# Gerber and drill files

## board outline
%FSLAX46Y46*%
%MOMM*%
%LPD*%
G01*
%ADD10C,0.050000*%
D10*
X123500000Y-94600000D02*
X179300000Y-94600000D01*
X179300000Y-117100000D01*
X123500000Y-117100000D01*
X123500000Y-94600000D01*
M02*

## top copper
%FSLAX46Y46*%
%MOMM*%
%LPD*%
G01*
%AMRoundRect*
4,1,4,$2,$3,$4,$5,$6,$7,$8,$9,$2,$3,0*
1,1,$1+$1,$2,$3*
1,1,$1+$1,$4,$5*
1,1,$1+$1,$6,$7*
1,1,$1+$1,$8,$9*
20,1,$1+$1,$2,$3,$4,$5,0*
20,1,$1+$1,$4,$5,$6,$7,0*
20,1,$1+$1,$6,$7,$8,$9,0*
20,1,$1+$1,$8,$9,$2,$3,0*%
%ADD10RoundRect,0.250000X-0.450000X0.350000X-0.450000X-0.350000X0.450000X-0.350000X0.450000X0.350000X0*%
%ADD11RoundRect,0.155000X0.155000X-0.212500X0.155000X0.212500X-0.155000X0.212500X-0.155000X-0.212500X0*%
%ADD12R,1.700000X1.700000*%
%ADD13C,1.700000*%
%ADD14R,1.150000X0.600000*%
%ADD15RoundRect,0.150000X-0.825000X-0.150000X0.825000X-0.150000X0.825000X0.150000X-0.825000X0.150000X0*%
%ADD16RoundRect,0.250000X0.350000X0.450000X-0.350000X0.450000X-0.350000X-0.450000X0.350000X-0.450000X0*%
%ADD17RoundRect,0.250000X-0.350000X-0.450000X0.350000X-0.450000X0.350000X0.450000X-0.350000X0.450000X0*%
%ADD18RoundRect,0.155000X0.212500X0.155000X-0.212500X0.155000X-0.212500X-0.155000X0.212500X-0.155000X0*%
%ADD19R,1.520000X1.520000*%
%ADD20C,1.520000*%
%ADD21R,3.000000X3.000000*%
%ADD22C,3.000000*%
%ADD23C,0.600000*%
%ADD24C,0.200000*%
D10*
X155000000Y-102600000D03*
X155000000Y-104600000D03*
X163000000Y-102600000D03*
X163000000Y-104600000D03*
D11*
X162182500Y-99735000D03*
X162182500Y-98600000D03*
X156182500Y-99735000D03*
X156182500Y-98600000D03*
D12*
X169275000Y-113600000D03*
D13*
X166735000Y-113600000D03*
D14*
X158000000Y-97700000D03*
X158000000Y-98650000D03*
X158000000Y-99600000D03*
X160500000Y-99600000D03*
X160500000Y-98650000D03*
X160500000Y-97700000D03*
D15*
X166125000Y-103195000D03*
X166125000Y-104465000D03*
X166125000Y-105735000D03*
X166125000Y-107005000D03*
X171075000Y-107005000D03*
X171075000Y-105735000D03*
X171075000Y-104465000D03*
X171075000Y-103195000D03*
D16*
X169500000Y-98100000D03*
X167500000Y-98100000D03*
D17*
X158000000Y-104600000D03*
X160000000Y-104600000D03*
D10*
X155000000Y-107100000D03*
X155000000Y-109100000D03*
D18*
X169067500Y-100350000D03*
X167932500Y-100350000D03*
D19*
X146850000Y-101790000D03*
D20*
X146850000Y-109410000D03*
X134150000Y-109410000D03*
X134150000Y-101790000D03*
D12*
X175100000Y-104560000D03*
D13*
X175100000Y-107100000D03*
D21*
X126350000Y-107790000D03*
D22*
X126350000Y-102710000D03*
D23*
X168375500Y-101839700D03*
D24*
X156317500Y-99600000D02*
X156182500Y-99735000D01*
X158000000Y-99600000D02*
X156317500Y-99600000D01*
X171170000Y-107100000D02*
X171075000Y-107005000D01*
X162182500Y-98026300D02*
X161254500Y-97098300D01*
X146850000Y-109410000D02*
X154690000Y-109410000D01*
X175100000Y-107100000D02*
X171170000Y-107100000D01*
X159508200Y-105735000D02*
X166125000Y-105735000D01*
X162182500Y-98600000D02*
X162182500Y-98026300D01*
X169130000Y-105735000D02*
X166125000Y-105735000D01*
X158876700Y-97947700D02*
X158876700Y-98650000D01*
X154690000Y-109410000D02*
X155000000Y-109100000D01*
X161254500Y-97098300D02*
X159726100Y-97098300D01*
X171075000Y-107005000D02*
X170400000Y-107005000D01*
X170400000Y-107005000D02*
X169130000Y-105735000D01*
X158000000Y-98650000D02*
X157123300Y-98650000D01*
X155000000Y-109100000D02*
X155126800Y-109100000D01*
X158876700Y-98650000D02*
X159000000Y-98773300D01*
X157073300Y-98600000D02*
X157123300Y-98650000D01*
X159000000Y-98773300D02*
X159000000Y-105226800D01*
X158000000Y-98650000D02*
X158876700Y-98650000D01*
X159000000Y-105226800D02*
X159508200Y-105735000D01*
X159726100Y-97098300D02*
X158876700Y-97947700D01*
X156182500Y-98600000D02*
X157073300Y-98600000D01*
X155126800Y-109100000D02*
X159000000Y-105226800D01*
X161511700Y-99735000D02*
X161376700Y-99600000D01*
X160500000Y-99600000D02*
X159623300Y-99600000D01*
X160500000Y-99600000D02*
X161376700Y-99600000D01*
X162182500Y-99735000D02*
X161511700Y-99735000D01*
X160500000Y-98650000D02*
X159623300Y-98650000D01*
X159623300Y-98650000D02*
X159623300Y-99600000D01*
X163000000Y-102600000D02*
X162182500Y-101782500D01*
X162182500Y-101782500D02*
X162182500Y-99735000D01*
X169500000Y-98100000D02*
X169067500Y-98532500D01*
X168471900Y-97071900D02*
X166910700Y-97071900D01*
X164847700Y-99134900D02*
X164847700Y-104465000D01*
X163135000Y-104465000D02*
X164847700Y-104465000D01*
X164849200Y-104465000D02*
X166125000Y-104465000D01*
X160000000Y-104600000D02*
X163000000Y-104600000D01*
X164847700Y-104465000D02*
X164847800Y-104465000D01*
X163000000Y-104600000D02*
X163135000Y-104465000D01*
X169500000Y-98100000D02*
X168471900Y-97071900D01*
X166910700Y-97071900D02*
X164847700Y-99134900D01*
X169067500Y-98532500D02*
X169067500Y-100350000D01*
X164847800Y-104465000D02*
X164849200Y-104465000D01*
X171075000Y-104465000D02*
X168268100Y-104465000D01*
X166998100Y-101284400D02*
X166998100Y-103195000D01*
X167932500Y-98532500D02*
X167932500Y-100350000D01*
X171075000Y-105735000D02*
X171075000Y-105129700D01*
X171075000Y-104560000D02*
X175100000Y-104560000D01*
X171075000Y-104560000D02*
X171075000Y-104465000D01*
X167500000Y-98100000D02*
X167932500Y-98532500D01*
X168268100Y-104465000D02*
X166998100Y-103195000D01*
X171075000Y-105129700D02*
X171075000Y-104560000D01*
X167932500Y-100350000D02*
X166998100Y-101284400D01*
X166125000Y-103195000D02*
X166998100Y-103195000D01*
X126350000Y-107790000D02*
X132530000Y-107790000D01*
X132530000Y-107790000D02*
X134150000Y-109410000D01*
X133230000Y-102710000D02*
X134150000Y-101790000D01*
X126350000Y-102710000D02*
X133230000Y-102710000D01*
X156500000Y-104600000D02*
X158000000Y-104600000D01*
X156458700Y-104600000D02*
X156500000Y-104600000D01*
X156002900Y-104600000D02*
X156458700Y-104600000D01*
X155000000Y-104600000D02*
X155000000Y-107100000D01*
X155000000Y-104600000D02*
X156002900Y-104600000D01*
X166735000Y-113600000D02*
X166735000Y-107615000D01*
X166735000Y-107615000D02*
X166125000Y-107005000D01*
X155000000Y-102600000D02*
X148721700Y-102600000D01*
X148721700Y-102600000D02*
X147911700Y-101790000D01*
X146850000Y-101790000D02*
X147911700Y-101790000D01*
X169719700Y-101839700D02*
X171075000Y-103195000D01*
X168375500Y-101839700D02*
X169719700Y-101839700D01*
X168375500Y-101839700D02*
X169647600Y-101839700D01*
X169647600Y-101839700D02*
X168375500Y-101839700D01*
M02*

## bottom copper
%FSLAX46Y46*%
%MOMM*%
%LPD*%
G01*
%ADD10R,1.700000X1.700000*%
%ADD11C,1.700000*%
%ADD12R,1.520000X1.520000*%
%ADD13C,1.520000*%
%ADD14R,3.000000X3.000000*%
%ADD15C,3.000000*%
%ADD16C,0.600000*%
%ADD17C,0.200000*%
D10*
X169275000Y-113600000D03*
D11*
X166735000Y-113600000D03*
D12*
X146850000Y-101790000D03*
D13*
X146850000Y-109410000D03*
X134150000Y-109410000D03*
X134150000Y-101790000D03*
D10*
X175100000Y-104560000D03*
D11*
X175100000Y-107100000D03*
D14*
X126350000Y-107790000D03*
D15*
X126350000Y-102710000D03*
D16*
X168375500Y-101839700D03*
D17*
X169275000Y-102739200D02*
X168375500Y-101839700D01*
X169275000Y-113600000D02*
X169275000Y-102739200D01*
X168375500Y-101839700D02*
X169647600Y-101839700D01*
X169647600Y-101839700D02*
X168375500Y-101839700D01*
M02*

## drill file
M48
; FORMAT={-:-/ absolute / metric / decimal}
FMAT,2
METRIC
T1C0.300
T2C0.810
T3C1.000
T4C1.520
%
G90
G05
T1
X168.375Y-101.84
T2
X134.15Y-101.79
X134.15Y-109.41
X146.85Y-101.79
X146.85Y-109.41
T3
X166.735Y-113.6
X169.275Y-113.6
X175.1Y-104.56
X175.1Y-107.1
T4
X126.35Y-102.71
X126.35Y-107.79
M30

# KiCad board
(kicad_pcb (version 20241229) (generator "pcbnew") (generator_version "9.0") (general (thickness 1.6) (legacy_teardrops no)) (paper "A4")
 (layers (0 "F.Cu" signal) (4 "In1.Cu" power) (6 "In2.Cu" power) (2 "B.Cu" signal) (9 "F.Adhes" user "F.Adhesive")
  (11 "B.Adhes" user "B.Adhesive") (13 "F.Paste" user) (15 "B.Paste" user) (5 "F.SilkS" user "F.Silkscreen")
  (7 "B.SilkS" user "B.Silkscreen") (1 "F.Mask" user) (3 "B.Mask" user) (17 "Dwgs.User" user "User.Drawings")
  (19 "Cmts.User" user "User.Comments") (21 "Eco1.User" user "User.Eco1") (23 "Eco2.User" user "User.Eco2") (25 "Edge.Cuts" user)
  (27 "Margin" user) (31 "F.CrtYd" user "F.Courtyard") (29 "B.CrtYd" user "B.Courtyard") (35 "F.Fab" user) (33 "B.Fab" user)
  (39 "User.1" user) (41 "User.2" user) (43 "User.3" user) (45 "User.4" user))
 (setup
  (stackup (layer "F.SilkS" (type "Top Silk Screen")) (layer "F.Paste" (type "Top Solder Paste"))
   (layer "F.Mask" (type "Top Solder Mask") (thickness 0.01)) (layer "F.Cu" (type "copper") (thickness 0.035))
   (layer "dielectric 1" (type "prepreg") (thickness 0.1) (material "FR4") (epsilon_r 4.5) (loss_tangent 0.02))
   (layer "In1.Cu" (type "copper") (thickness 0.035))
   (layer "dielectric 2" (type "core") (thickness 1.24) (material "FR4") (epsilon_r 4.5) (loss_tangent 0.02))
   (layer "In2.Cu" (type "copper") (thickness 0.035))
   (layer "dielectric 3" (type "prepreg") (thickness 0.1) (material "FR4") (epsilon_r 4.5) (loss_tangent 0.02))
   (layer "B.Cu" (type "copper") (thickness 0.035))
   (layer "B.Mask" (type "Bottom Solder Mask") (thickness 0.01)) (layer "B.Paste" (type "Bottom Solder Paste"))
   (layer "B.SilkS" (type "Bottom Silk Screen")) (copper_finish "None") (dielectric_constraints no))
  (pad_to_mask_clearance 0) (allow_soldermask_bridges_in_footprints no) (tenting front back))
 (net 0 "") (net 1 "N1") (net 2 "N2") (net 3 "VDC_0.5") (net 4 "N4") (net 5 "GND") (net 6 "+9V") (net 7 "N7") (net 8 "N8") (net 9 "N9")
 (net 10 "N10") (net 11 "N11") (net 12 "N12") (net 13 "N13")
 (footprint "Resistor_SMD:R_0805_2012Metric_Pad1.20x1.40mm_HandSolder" (layer "F.Cu") (at 155 103.6 -90)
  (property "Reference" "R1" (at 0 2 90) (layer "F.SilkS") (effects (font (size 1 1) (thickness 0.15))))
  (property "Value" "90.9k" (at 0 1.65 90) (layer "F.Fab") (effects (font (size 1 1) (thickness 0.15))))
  (pad "1" smd roundrect (at -1 0 270) (size 1.2 1.4) (layers "F.Cu" "F.Mask" "F.Paste") (roundrect_rratio 0.208333) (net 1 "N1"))
  (pad "2" smd roundrect (at 1 0 270) (size 1.2 1.4) (layers "F.Cu" "F.Mask" "F.Paste") (roundrect_rratio 0.208333) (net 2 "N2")))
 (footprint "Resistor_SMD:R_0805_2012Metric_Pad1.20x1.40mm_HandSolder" (layer "F.Cu") (at 163 103.6 -90)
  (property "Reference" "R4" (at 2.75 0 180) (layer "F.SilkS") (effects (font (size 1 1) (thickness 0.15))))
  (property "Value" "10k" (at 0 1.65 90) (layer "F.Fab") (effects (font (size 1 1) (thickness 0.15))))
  (pad "1" smd roundrect (at -1 0 270) (size 1.2 1.4) (layers "F.Cu" "F.Mask" "F.Paste") (roundrect_rratio 0.208333) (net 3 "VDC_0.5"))
  (pad "2" smd roundrect (at 1 0 270) (size 1.2 1.4) (layers "F.Cu" "F.Mask" "F.Paste") (roundrect_rratio 0.208333) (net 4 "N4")))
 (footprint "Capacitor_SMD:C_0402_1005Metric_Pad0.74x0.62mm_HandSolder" (layer "F.Cu") (at 162.1825 99.1675 90)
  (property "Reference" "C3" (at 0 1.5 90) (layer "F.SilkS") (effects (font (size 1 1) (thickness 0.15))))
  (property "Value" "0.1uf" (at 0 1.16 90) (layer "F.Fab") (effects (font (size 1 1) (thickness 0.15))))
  (pad "1" smd roundrect (at -0.5675 0 90) (size 0.735 0.62) (layers "F.Cu" "F.Mask" "F.Paste") (roundrect_rratio 0.25) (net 3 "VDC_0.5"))
  (pad "2" smd roundrect (at 0.5675 0 90) (size 0.735 0.62) (layers "F.Cu" "F.Mask" "F.Paste") (roundrect_rratio 0.25) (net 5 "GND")))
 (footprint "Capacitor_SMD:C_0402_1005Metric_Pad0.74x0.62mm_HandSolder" (layer "F.Cu") (at 156.1825 99.1675 90)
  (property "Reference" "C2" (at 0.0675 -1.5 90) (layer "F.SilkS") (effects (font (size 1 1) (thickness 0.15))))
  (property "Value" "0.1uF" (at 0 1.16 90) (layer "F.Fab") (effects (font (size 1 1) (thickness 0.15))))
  (pad "1" smd roundrect (at -0.5675 0 90) (size 0.735 0.62) (layers "F.Cu" "F.Mask" "F.Paste") (roundrect_rratio 0.25) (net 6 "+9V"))
  (pad "2" smd roundrect (at 0.5675 0 90) (size 0.735 0.62) (layers "F.Cu" "F.Mask" "F.Paste") (roundrect_rratio 0.25) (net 5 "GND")))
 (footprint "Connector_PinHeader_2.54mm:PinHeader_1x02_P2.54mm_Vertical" (layer "F.Cu") (at 169.275 113.6 -90)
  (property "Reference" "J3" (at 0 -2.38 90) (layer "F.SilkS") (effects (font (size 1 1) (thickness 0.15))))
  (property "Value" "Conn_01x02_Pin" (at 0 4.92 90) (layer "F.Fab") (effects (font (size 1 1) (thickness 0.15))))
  (pad "1" thru_hole rect (at 0 0 270) (size 1.7 1.7) (drill 1) (layers "*.Cu" "*.Mask") (remove_unused_layers no) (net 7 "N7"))
  (pad "2" thru_hole circle (at 0 2.54 270) (size 1.7 1.7) (drill 1) (layers "*.Cu" "*.Mask") (remove_unused_layers no) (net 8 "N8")))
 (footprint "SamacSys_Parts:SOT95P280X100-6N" (layer "F.Cu") (at 159.25 98.65)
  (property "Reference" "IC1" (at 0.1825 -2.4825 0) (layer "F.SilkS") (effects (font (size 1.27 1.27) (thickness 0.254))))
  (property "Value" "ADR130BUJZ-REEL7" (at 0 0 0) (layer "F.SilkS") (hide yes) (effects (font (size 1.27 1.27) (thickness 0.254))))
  (pad "1" smd rect (at -1.25 -0.95 90) (size 0.6 1.15) (layers "F.Cu" "F.Mask" "F.Paste") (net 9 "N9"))
  (pad "2" smd rect (at -1.25 0 90) (size 0.6 1.15) (layers "F.Cu" "F.Mask" "F.Paste") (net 5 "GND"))
  (pad "3" smd rect (at -1.25 0.95 90) (size 0.6 1.15) (layers "F.Cu" "F.Mask" "F.Paste") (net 6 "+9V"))
  (pad "4" smd rect (at 1.25 0.95 90) (size 0.6 1.15) (layers "F.Cu" "F.Mask" "F.Paste") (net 3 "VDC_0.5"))
  (pad "5" smd rect (at 1.25 0 90) (size 0.6 1.15) (layers "F.Cu" "F.Mask" "F.Paste") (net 3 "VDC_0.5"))
  (pad "6" smd rect (at 1.25 -0.95 90) (size 0.6 1.15) (layers "F.Cu" "F.Mask" "F.Paste") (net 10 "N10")))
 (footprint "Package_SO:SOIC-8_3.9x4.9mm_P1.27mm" (layer "F.Cu") (at 168.6 105.1)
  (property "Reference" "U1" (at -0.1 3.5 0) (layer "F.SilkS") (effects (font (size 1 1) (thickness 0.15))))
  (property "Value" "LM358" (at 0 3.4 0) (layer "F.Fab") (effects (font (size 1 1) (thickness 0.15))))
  (pad "1" smd roundrect (at -2.475 -1.905) (size 1.95 0.6) (layers "F.Cu" "F.Mask" "F.Paste") (roundrect_rratio 0.25) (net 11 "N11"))
  (pad "2" smd roundrect (at -2.475 -0.635) (size 1.95 0.6) (layers "F.Cu" "F.Mask" "F.Paste") (roundrect_rratio 0.25) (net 4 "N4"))
  (pad "3" smd roundrect (at -2.475 0.635) (size 1.95 0.6) (layers "F.Cu" "F.Mask" "F.Paste") (roundrect_rratio 0.25) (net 5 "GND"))
  (pad "4" smd roundrect (at -2.475 1.905) (size 1.95 0.6) (layers "F.Cu" "F.Mask" "F.Paste") (roundrect_rratio 0.25) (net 8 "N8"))
  (pad "5" smd roundrect (at 2.475 1.905) (size 1.95 0.6) (layers "F.Cu" "F.Mask" "F.Paste") (roundrect_rratio 0.25) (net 5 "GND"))
  (pad "6" smd roundrect (at 2.475 0.635) (size 1.95 0.6) (layers "F.Cu" "F.Mask" "F.Paste") (roundrect_rratio 0.25) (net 11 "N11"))
  (pad "7" smd roundrect (at 2.475 -0.635) (size 1.95 0.6) (layers "F.Cu" "F.Mask" "F.Paste") (roundrect_rratio 0.25) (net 11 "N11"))
  (pad "8" smd roundrect (at 2.475 -1.905) (size 1.95 0.6) (layers "F.Cu" "F.Mask" "F.Paste") (roundrect_rratio 0.25) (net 7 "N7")))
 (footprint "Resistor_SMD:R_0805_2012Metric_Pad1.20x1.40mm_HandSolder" (layer "F.Cu") (at 168.5 98.1 180)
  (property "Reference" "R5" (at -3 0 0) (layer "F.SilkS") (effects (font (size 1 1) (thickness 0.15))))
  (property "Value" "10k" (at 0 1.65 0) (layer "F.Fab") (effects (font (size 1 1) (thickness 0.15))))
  (pad "1" smd roundrect (at -1 0 180) (size 1.2 1.4) (layers "F.Cu" "F.Mask" "F.Paste") (roundrect_rratio 0.208333) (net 4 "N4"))
  (pad "2" smd roundrect (at 1 0 180) (size 1.2 1.4) (layers "F.Cu" "F.Mask" "F.Paste") (roundrect_rratio 0.208333) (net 11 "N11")))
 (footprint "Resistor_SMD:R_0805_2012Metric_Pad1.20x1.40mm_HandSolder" (layer "F.Cu") (at 159 104.6)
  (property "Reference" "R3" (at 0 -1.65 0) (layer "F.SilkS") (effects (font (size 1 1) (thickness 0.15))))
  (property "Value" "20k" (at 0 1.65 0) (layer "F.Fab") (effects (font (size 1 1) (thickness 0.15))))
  (pad "1" smd roundrect (at -1 0) (size 1.2 1.4) (layers "F.Cu" "F.Mask" "F.Paste") (roundrect_rratio 0.208333) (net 2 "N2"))
  (pad "2" smd roundrect (at 1 0) (size 1.2 1.4) (layers "F.Cu" "F.Mask" "F.Paste") (roundrect_rratio 0.208333) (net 4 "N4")))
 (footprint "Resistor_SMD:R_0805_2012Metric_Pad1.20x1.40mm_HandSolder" (layer "F.Cu") (at 155 108.1 -90)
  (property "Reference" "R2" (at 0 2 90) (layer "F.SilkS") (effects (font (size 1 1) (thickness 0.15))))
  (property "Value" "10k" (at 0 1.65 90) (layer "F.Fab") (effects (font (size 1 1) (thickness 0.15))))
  (pad "1" smd roundrect (at -1 0 270) (size 1.2 1.4) (layers "F.Cu" "F.Mask" "F.Paste") (roundrect_rratio 0.208333) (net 2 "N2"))
  (pad "2" smd roundrect (at 1 0 270) (size 1.2 1.4) (layers "F.Cu" "F.Mask" "F.Paste") (roundrect_rratio 0.208333) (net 5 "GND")))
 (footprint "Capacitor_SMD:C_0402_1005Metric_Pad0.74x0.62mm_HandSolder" (layer "F.Cu") (at 168.5 100.35 180)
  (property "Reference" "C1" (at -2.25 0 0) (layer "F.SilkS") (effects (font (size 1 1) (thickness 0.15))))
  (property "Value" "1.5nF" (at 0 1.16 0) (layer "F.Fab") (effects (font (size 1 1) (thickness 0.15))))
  (pad "1" smd roundrect (at -0.5675 0 180) (size 0.735 0.62) (layers "F.Cu" "F.Mask" "F.Paste") (roundrect_rratio 0.25) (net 4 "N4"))
  (pad "2" smd roundrect (at 0.5675 0 180) (size 0.735 0.62) (layers "F.Cu" "F.Mask" "F.Paste") (roundrect_rratio 0.25) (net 11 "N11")))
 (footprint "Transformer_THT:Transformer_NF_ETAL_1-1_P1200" (layer "F.Cu") (at 146.85 101.79)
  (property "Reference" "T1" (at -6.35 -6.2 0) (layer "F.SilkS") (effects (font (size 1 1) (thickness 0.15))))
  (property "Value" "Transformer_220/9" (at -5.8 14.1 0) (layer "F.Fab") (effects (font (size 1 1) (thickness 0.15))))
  (pad "1" thru_hole rect (at 0 0) (size 1.52 1.52) (drill 0.81) (layers "*.Cu" "*.Mask") (remove_unused_layers no) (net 1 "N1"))
  (pad "3" thru_hole circle (at 0 7.62) (size 1.52 1.52) (drill 0.81) (layers "*.Cu" "*.Mask") (remove_unused_layers no) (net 5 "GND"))
  (pad "4" thru_hole circle (at -12.7 7.62) (size 1.52 1.52) (drill 0.81) (layers "*.Cu" "*.Mask") (remove_unused_layers no) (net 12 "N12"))
  (pad "6" thru_hole circle (at -12.7 0) (size 1.52 1.52) (drill 0.81) (layers "*.Cu" "*.Mask") (remove_unused_layers no) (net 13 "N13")))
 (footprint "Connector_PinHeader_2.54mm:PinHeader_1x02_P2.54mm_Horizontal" (layer "F.Cu") (at 175.1 104.56)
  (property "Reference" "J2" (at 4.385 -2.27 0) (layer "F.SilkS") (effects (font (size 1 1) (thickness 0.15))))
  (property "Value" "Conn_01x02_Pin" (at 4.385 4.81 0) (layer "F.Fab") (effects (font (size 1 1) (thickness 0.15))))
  (pad "1" thru_hole rect (at 0 0) (size 1.7 1.7) (drill 1) (layers "*.Cu" "*.Mask") (remove_unused_layers no) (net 11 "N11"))
  (pad "2" thru_hole circle (at 0 2.54) (size 1.7 1.7) (drill 1) (layers "*.Cu" "*.Mask") (remove_unused_layers no) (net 5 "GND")))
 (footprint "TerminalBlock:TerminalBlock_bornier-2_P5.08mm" (layer "F.Cu") (at 126.35 107.79 90)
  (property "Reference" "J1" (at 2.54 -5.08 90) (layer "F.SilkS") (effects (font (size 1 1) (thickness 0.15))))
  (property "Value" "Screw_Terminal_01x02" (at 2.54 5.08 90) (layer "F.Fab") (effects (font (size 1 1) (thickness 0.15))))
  (pad "1" thru_hole rect (at 0 0 90) (size 3 3) (drill 1.52) (layers "*.Cu" "*.Mask") (remove_unused_layers no) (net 12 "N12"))
  (pad "2" thru_hole circle (at 5.08 0 90) (size 3 3) (drill 1.52) (layers "*.Cu" "*.Mask") (remove_unused_layers no) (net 13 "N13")))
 (gr_rect (start 123.5 94.6) (end 179.3 117.1) (stroke (width 0.05) (type default)) (fill no) (layer "Edge.Cuts"))
 (segment (start 156.3175 99.6) (end 156.1825 99.735) (width 0.2) (layer "F.Cu") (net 6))
 (segment (start 158 99.6) (end 156.3175 99.6) (width 0.2) (layer "F.Cu") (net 6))
 (segment (start 171.17 107.1) (end 171.075 107.005) (width 0.2) (layer "F.Cu") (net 5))
 (segment (start 162.1825 98.0263) (end 161.2545 97.0983) (width 0.2) (layer "F.Cu") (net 5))
 (segment (start 146.85 109.41) (end 154.69 109.41) (width 0.2) (layer "F.Cu") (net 5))
 (segment (start 175.1 107.1) (end 171.17 107.1) (width 0.2) (layer "F.Cu") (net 5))
 (segment (start 159.5082 105.735) (end 166.125 105.735) (width 0.2) (layer "F.Cu") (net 5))
 (segment (start 162.1825 98.6) (end 162.1825 98.0263) (width 0.2) (layer "F.Cu") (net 5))
 (segment (start 169.13 105.735) (end 166.125 105.735) (width 0.2) (layer "F.Cu") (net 5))
 (segment (start 158.8767 97.9477) (end 158.8767 98.65) (width 0.2) (layer "F.Cu") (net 5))
 (segment (start 154.69 109.41) (end 155 109.1) (width 0.2) (layer "F.Cu") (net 5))
 (segment (start 161.2545 97.0983) (end 159.7261 97.0983) (width 0.2) (layer "F.Cu") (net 5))
 (segment (start 171.075 107.005) (end 170.4 107.005) (width 0.2) (layer "F.Cu") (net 5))
 (segment (start 170.4 107.005) (end 169.13 105.735) (width 0.2) (layer "F.Cu") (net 5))
 (segment (start 158 98.65) (end 157.1233 98.65) (width 0.2) (layer "F.Cu") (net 5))
 (segment (start 155 109.1) (end 155.1268 109.1) (width 0.2) (layer "F.Cu") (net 5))
 (segment (start 158.8767 98.65) (end 159 98.7733) (width 0.2) (layer "F.Cu") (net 5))
 (segment (start 157.0733 98.6) (end 157.1233 98.65) (width 0.2) (layer "F.Cu") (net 5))
 (segment (start 159 98.7733) (end 159 105.2268) (width 0.2) (layer "F.Cu") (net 5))
 (segment (start 158 98.65) (end 158.8767 98.65) (width 0.2) (layer "F.Cu") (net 5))
 (segment (start 159 105.2268) (end 159.5082 105.735) (width 0.2) (layer "F.Cu") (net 5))
 (segment (start 159.7261 97.0983) (end 158.8767 97.9477) (width 0.2) (layer "F.Cu") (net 5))
 (segment (start 156.1825 98.6) (end 157.0733 98.6) (width 0.2) (layer "F.Cu") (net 5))
 (segment (start 155.1268 109.1) (end 159 105.2268) (width 0.2) (layer "F.Cu") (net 5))
 (segment (start 161.5117 99.735) (end 161.3767 99.6) (width 0.2) (layer "F.Cu") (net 3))
 (segment (start 160.5 99.6) (end 159.6233 99.6) (width 0.2) (layer "F.Cu") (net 3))
 (segment (start 160.5 99.6) (end 161.3767 99.6) (width 0.2) (layer "F.Cu") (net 3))
 (segment (start 162.1825 99.735) (end 161.5117 99.735) (width 0.2) (layer "F.Cu") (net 3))
 (segment (start 160.5 98.65) (end 159.6233 98.65) (width 0.2) (layer "F.Cu") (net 3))
 (segment (start 159.6233 98.65) (end 159.6233 99.6) (width 0.2) (layer "F.Cu") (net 3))
 (segment (start 163 102.6) (end 162.1825 101.7825) (width 0.2) (layer "F.Cu") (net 3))
 (segment (start 162.1825 101.7825) (end 162.1825 99.735) (width 0.2) (layer "F.Cu") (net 3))
 (segment (start 169.5 98.1) (end 169.0675 98.5325) (width 0.2) (layer "F.Cu") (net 4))
 (segment (start 168.4719 97.0719) (end 166.9107 97.0719) (width 0.2) (layer "F.Cu") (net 4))
 (segment (start 164.8477 99.1349) (end 164.8477 104.465) (width 0.2) (layer "F.Cu") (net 4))
 (segment (start 163.135 104.465) (end 164.8477 104.465) (width 0.2) (layer "F.Cu") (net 4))
 (segment (start 164.8492 104.465) (end 166.125 104.465) (width 0.2) (layer "F.Cu") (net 4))
 (segment (start 160 104.6) (end 163 104.6) (width 0.2) (layer "F.Cu") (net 4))
 (segment (start 164.8477 104.465) (end 164.8478 104.465) (width 0.2) (layer "F.Cu") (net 4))
 (segment (start 163 104.6) (end 163.135 104.465) (width 0.2) (layer "F.Cu") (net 4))
 (segment (start 169.5 98.1) (end 168.4719 97.0719) (width 0.2) (layer "F.Cu") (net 4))
 (segment (start 166.9107 97.0719) (end 164.8477 99.1349) (width 0.2) (layer "F.Cu") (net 4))
 (segment (start 169.0675 98.5325) (end 169.0675 100.35) (width 0.2) (layer "F.Cu") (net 4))
 (segment (start 164.8478 104.465) (end 164.8492 104.465) (width 0.2) (layer "F.Cu") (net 4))
 (segment (start 171.075 104.465) (end 168.2681 104.465) (width 0.2) (layer "F.Cu") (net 11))
 (segment (start 166.9981 101.2844) (end 166.9981 103.195) (width 0.2) (layer "F.Cu") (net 11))
 (segment (start 167.9325 98.5325) (end 167.9325 100.35) (width 0.2) (layer "F.Cu") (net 11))
 (segment (start 171.075 105.735) (end 171.075 105.1297) (width 0.2) (layer "F.Cu") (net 11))
 (segment (start 171.075 104.56) (end 175.1 104.56) (width 0.2) (layer "F.Cu") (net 11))
 (segment (start 171.075 104.56) (end 171.075 104.465) (width 0.2) (layer "F.Cu") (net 11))
 (segment (start 167.5 98.1) (end 167.9325 98.5325) (width 0.2) (layer "F.Cu") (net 11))
 (segment (start 168.2681 104.465) (end 166.9981 103.195) (width 0.2) (layer "F.Cu") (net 11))
 (segment (start 171.075 105.1297) (end 171.075 104.56) (width 0.2) (layer "F.Cu") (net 11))
 (segment (start 167.9325 100.35) (end 166.9981 101.2844) (width 0.2) (layer "F.Cu") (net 11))
 (segment (start 166.125 103.195) (end 166.9981 103.195) (width 0.2) (layer "F.Cu") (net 11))
 (segment (start 126.35 107.79) (end 132.53 107.79) (width 0.2) (layer "F.Cu") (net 12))
 (segment (start 132.53 107.79) (end 134.15 109.41) (width 0.2) (layer "F.Cu") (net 12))
 (segment (start 133.23 102.71) (end 134.15 101.79) (width 0.2) (layer "F.Cu") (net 13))
 (segment (start 126.35 102.71) (end 133.23 102.71) (width 0.2) (layer "F.Cu") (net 13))
 (segment (start 156.5 104.6) (end 158 104.6) (width 0.2) (layer "F.Cu") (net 2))
 (segment (start 156.4587 104.6) (end 156.5 104.6) (width 0.2) (layer "F.Cu") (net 2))
 (segment (start 156.0029 104.6) (end 156.4587 104.6) (width 0.2) (layer "F.Cu") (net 2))
 (segment (start 155 104.6) (end 155 107.1) (width 0.2) (layer "F.Cu") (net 2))
 (segment (start 155 104.6) (end 156.0029 104.6) (width 0.2) (layer "F.Cu") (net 2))
 (segment (start 166.735 113.6) (end 166.735 107.615) (width 0.2) (layer "F.Cu") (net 8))
 (segment (start 166.735 107.615) (end 166.125 107.005) (width 0.2) (layer "F.Cu") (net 8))
 (segment (start 155 102.6) (end 148.7217 102.6) (width 0.2) (layer "F.Cu") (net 1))
 (segment (start 148.7217 102.6) (end 147.9117 101.79) (width 0.2) (layer "F.Cu") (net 1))
 (segment (start 146.85 101.79) (end 147.9117 101.79) (width 0.2) (layer "F.Cu") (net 1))
 (segment (start 169.7197 101.8397) (end 171.075 103.195) (width 0.2) (layer "F.Cu") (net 7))
 (segment (start 168.3755 101.8397) (end 169.7197 101.8397) (width 0.2) (layer "F.Cu") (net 7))
 (segment (start 168.3755 101.8397) (end 169.6476 101.8397) (width 0.2) (layer "F.Cu") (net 7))
 (segment (start 169.6476 101.8397) (end 168.3755 101.8397) (width 0.2) (layer "F.Cu") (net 7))
 (via (at 168.3755 101.8397) (size 0.6) (drill 0.3) (layers "F.Cu" "B.Cu") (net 7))
 (segment (start 169.275 102.7392) (end 168.3755 101.8397) (width 0.2) (layer "B.Cu") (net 7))
 (segment (start 169.275 113.6) (end 169.275 102.7392) (width 0.2) (layer "B.Cu") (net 7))
 (segment (start 168.3755 101.8397) (end 169.6476 101.8397) (width 0.2) (layer "B.Cu") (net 7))
 (segment (start 169.6476 101.8397) (end 168.3755 101.8397) (width 0.2) (layer "B.Cu") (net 7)))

